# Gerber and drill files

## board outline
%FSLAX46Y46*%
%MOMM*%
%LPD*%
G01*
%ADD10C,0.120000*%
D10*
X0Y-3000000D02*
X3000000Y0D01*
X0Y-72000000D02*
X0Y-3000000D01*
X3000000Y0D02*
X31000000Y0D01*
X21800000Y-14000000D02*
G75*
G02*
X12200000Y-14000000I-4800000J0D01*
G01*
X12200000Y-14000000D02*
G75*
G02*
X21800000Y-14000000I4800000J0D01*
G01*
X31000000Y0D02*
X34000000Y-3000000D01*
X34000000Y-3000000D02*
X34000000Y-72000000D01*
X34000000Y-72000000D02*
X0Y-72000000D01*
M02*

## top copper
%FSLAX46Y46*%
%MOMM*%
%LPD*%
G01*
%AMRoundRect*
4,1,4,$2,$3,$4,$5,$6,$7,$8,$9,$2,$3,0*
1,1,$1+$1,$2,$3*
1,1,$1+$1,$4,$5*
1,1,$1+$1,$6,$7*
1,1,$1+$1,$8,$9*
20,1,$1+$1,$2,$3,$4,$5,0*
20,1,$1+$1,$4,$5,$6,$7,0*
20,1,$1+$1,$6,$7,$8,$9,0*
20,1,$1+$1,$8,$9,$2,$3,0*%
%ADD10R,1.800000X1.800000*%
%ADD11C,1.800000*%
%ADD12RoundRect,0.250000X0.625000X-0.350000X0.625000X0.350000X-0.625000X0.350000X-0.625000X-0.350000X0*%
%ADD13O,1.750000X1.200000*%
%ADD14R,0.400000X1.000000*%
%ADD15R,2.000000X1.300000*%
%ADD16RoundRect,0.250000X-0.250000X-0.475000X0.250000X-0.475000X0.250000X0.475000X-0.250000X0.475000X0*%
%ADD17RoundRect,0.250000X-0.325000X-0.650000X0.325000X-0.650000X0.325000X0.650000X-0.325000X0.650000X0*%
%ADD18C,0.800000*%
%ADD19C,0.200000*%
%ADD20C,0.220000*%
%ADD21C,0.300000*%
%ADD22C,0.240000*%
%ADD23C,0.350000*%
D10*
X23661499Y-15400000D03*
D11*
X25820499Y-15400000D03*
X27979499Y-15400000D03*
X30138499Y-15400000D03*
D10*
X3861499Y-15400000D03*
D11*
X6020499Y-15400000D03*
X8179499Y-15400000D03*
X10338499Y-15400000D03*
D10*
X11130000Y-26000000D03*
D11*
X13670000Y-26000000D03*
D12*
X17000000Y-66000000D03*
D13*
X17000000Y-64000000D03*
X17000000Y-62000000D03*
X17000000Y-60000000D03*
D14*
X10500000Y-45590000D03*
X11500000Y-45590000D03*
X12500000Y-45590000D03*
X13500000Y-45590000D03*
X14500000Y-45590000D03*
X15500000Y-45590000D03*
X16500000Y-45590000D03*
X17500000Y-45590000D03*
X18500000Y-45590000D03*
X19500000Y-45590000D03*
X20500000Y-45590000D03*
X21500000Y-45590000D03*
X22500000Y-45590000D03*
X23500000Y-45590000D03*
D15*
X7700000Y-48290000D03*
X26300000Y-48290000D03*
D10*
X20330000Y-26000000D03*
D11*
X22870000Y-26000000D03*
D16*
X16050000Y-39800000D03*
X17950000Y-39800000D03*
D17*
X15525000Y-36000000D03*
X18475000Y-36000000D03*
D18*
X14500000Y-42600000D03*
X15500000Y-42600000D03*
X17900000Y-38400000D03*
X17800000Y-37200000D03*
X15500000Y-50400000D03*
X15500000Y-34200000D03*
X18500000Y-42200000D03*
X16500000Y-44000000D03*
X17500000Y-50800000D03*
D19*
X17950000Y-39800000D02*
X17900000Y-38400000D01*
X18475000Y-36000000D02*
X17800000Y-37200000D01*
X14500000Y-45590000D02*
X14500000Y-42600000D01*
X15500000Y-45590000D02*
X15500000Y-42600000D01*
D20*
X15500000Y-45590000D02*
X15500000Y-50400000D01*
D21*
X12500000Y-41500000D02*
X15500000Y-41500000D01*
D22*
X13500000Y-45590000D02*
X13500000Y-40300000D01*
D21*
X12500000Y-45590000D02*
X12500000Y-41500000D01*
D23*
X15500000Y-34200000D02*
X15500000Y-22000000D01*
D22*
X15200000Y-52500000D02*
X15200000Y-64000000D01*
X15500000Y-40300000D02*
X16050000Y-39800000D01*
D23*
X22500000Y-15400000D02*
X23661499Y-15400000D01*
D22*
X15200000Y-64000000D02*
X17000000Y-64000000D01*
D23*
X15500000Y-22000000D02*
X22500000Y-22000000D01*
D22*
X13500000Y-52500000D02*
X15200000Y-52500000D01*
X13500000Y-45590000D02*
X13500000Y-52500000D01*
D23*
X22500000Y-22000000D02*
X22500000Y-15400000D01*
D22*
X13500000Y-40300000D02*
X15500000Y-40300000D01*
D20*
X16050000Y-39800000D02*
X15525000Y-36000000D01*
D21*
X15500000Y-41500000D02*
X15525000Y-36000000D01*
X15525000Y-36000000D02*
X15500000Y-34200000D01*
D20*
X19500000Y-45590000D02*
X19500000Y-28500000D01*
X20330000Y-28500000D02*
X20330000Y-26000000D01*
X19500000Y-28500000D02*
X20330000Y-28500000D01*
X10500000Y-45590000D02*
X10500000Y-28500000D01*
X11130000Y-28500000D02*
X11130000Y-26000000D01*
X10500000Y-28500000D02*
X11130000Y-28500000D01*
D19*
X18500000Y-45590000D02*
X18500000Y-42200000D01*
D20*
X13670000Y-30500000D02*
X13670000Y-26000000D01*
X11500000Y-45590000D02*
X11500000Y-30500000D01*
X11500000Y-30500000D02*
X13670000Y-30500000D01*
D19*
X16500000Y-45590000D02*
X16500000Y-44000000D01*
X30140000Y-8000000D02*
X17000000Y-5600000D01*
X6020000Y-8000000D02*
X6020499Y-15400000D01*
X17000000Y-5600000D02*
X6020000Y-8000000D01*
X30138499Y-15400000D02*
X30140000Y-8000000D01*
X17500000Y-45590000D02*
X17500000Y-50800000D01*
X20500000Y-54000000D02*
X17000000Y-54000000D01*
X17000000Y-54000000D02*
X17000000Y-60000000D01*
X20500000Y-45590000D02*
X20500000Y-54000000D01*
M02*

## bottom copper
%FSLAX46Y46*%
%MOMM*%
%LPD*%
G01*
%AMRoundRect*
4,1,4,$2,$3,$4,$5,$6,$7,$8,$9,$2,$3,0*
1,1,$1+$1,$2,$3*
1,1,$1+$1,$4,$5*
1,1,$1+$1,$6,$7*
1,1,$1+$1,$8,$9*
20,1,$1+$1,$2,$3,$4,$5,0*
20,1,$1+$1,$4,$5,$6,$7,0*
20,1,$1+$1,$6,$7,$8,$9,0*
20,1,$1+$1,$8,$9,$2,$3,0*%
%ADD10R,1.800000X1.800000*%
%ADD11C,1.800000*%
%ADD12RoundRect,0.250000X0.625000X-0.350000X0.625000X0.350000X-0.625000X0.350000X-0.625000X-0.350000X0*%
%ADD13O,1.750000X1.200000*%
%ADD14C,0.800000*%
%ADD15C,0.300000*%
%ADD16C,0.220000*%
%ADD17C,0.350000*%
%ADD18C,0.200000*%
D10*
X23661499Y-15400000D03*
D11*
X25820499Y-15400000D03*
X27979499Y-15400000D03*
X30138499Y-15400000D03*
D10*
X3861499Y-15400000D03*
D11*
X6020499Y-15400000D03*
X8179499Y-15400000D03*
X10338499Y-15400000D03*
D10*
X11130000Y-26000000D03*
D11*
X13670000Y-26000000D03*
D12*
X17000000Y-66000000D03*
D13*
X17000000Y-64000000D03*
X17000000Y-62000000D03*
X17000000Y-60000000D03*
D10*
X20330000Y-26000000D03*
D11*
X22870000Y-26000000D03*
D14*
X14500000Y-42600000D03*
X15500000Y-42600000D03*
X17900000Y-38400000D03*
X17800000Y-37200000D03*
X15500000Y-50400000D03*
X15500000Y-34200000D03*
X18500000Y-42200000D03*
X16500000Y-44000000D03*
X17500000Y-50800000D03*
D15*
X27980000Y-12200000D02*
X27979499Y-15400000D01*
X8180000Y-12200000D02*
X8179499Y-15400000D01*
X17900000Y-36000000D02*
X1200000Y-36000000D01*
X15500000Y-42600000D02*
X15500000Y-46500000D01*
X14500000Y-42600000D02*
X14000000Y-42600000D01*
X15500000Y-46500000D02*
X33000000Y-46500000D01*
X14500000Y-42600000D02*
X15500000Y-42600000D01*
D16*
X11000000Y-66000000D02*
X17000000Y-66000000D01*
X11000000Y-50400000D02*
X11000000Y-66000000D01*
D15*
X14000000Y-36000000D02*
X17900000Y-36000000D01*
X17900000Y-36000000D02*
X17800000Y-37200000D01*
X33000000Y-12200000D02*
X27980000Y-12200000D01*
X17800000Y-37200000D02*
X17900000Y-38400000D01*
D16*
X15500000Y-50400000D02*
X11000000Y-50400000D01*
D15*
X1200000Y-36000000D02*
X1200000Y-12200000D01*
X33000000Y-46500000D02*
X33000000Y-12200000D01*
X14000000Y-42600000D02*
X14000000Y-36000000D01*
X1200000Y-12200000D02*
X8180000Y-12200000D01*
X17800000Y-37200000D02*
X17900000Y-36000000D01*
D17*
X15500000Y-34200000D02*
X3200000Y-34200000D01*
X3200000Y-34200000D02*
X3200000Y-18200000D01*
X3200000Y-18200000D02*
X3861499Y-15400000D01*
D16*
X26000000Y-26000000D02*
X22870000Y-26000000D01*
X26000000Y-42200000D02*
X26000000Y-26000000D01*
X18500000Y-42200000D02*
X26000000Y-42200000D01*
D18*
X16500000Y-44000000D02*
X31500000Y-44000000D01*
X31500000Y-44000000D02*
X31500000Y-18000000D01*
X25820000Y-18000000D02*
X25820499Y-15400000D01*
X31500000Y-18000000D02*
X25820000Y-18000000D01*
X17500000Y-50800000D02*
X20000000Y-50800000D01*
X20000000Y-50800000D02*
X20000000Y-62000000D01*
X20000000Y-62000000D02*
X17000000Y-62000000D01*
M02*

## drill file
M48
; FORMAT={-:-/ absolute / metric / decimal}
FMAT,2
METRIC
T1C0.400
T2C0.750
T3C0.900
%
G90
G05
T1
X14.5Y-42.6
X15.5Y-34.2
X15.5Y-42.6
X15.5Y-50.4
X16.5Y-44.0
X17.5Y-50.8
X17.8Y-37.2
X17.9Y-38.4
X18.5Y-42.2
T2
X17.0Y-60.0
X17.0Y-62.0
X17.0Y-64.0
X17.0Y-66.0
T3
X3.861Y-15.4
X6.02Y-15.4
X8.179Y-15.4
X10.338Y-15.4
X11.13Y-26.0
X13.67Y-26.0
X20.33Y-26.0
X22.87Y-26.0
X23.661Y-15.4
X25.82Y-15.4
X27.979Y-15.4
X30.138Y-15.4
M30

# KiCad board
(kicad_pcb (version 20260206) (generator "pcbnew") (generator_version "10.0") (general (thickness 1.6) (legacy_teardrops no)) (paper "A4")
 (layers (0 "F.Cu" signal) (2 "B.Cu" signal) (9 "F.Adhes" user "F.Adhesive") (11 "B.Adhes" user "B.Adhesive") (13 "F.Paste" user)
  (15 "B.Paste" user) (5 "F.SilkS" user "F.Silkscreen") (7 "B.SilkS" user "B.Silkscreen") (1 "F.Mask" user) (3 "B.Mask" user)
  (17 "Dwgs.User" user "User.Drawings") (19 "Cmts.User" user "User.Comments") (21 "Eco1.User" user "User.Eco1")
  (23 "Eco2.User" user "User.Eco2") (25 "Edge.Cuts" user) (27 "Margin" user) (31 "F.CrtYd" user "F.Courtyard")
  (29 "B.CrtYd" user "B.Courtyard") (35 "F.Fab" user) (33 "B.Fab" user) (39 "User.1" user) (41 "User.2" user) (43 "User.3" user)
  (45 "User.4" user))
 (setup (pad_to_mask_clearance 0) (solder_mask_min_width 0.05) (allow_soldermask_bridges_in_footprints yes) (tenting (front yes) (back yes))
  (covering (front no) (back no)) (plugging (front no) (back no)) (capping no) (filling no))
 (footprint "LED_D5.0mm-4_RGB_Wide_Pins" (layer "F.Cu") (at 23.661499 15.4)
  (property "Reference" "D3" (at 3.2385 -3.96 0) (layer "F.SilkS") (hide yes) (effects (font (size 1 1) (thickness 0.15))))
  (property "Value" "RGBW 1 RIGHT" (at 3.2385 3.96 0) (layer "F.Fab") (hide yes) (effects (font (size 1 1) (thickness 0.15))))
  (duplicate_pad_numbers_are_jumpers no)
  (pad "1" thru_hole rect (at 0 0) (size 1.8 1.8) (drill 0.9) (layers "*.Cu" "*.Mask") (remove_unused_layers no) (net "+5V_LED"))
  (pad "2" thru_hole circle (at 2.159 0) (size 1.8 1.8) (drill 0.9) (layers "*.Cu" "*.Mask") (remove_unused_layers no) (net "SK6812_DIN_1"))
  (pad "3" thru_hole circle (at 4.318 0) (size 1.8 1.8) (drill 0.9) (layers "*.Cu" "*.Mask") (remove_unused_layers no) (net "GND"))
  (pad "4" thru_hole circle (at 6.477 0) (size 1.8 1.8) (drill 0.9) (layers "*.Cu" "*.Mask") (remove_unused_layers no) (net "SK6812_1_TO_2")))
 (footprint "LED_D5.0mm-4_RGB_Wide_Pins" (layer "F.Cu") (at 3.861499 15.4)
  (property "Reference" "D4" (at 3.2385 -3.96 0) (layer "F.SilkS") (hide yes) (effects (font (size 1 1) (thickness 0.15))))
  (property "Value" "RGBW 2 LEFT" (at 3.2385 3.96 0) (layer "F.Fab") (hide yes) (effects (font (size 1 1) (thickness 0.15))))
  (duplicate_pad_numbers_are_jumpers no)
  (pad "1" thru_hole rect (at 0 0) (size 1.8 1.8) (drill 0.9) (layers "*.Cu" "*.Mask") (remove_unused_layers no) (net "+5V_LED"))
  (pad "2" thru_hole circle (at 2.159 0) (size 1.8 1.8) (drill 0.9) (layers "*.Cu" "*.Mask") (remove_unused_layers no) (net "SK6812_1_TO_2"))
  (pad "3" thru_hole circle (at 4.318 0) (size 1.8 1.8) (drill 0.9) (layers "*.Cu" "*.Mask") (remove_unused_layers no) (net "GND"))
  (pad "4" thru_hole circle (at 6.477 0) (size 1.8 1.8) (drill 0.9) (layers "*.Cu" "*.Mask") (remove_unused_layers no)))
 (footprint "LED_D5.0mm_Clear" (layer "F.Cu") (at 11.13 26)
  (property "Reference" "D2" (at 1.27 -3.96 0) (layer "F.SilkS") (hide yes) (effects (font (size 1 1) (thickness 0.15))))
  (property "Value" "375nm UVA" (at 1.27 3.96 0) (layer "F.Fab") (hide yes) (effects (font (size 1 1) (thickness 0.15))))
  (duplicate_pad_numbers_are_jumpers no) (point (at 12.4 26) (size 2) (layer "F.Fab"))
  (pad "1" thru_hole rect (at 0 0) (size 1.8 1.8) (drill 0.9) (layers "*.Cu" "*.Mask") (remove_unused_layers no) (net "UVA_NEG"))
  (pad "2" thru_hole circle (at 2.54 0) (size 1.8 1.8) (drill 0.9) (layers "*.Cu" "*.Mask") (remove_unused_layers no) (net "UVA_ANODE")))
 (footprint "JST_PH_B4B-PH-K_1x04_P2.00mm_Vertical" (layer "F.Cu") (at 17 66 90)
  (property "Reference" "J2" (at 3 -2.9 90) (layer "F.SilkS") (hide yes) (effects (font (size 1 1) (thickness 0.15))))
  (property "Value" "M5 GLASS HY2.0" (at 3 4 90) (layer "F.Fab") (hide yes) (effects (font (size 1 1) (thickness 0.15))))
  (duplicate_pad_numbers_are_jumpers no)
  (pad "1" thru_hole roundrect (at 0 0 90) (size 1.2 1.75) (drill 0.75) (layers "*.Cu" "*.Mask") (remove_unused_layers no)
   (roundrect_rratio 0.208333) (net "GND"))
  (pad "2" thru_hole oval (at 2 0 90) (size 1.2 1.75) (drill 0.75) (layers "*.Cu" "*.Mask") (remove_unused_layers no) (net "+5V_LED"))
  (pad "3" thru_hole oval (at 4 0 90) (size 1.2 1.75) (drill 0.75) (layers "*.Cu" "*.Mask") (remove_unused_layers no) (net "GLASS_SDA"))
  (pad "4" thru_hole oval (at 6 0 90) (size 1.2 1.75) (drill 0.75) (layers "*.Cu" "*.Mask") (remove_unused_layers no) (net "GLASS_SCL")))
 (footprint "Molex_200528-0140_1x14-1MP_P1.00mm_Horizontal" (layer "F.Cu") (at 17 46.5)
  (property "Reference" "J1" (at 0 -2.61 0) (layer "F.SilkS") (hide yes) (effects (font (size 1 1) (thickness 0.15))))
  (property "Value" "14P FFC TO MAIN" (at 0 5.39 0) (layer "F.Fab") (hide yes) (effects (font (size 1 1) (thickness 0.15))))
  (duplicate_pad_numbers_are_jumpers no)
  (pad "1" smd rect (at -6.5 -0.91) (size 0.4 1) (layers "F.Cu" "F.Mask" "F.Paste") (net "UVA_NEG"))
  (pad "2" smd rect (at -5.5 -0.91) (size 0.4 1) (layers "F.Cu" "F.Mask" "F.Paste") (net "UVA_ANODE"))
  (pad "3" smd rect (at -4.5 -0.91) (size 0.4 1) (layers "F.Cu" "F.Mask" "F.Paste") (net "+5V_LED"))
  (pad "4" smd rect (at -3.5 -0.91) (size 0.4 1) (layers "F.Cu" "F.Mask" "F.Paste") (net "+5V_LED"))
  (pad "5" smd rect (at -2.5 -0.91) (size 0.4 1) (layers "F.Cu" "F.Mask" "F.Paste") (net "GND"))
  (pad "6" smd rect (at -1.5 -0.91) (size 0.4 1) (layers "F.Cu" "F.Mask" "F.Paste") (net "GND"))
  (pad "7" smd rect (at -0.5 -0.91) (size 0.4 1) (layers "F.Cu" "F.Mask" "F.Paste") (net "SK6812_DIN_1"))
  (pad "8" smd rect (at 0.5 -0.91) (size 0.4 1) (layers "F.Cu" "F.Mask" "F.Paste") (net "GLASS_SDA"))
  (pad "9" smd rect (at 1.5 -0.91) (size 0.4 1) (layers "F.Cu" "F.Mask" "F.Paste") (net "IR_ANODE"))
  (pad "10" smd rect (at 2.5 -0.91) (size 0.4 1) (layers "F.Cu" "F.Mask" "F.Paste") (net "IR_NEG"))
  (pad "11" smd rect (at 3.5 -0.91) (size 0.4 1) (layers "F.Cu" "F.Mask" "F.Paste") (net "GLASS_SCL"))
  (pad "12" smd rect (at 4.5 -0.91) (size 0.4 1) (layers "F.Cu" "F.Mask" "F.Paste"))
  (pad "13" smd rect (at 5.5 -0.91) (size 0.4 1) (layers "F.Cu" "F.Mask" "F.Paste"))
  (pad "14" smd rect (at 6.5 -0.91) (size 0.4 1) (layers "F.Cu" "F.Mask" "F.Paste"))
  (pad "MP" smd rect (at -9.3 1.79) (size 2 1.3) (layers "F.Cu" "F.Mask" "F.Paste"))
  (pad "MP" smd rect (at 9.3 1.79) (size 2 1.3) (layers "F.Cu" "F.Mask" "F.Paste")))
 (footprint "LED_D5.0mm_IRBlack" (layer "F.Cu") (at 20.33 26)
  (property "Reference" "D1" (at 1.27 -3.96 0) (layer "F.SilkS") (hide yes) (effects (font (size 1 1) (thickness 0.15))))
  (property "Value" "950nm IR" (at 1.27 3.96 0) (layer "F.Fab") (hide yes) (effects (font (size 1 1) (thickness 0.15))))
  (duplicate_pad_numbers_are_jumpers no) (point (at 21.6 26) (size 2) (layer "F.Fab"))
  (pad "1" thru_hole rect (at 0 0) (size 1.8 1.8) (drill 0.9) (layers "*.Cu" "*.Mask") (remove_unused_layers no) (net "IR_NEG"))
  (pad "2" thru_hole circle (at 2.54 0) (size 1.8 1.8) (drill 0.9) (layers "*.Cu" "*.Mask") (remove_unused_layers no) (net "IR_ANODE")))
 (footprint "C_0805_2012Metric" (layer "F.Cu") (at 17 39.8)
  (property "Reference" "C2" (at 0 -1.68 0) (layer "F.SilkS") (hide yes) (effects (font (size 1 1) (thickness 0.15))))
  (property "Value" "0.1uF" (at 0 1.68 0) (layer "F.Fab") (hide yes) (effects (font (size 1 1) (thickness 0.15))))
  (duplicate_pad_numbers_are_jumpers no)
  (pad "1" smd roundrect (at -0.95 0) (size 1 1.45) (layers "F.Cu" "F.Mask" "F.Paste") (roundrect_rratio 0.25) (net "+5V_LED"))
  (pad "2" smd roundrect (at 0.95 0) (size 1 1.45) (layers "F.Cu" "F.Mask" "F.Paste") (roundrect_rratio 0.25) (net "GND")))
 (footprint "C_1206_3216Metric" (layer "F.Cu") (at 17 36)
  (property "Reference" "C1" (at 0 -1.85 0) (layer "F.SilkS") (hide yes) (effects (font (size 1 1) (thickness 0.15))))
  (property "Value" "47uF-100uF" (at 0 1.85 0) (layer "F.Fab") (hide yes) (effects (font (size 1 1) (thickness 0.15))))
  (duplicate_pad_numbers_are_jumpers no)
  (pad "1" smd roundrect (at -1.475 0) (size 1.15 1.8) (layers "F.Cu" "F.Mask" "F.Paste") (roundrect_rratio 0.217391) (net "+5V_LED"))
  (pad "2" smd roundrect (at 1.475 0) (size 1.15 1.8) (layers "F.Cu" "F.Mask" "F.Paste") (roundrect_rratio 0.217391) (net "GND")))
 (gr_line (start 0 3) (end 3 0) (stroke (width 0.12) (type default)) (layer "Edge.Cuts"))
 (gr_line (start 0 72) (end 0 3) (stroke (width 0.12) (type default)) (layer "Edge.Cuts"))
 (gr_line (start 3 0) (end 31 0) (stroke (width 0.12) (type default)) (layer "Edge.Cuts"))
 (gr_circle (center 17 14) (end 21.8 14) (stroke (width 0.12) (type default)) (fill no) (layer "Edge.Cuts"))
 (gr_line (start 31 0) (end 34 3) (stroke (width 0.12) (type default)) (layer "Edge.Cuts"))
 (gr_line (start 34 3) (end 34 72) (stroke (width 0.12) (type default)) (layer "Edge.Cuts"))
 (gr_line (start 34 72) (end 0 72) (stroke (width 0.12) (type default)) (layer "Edge.Cuts"))
 (segment (start 17.95 39.8) (end 17.9 38.4) (width 0.2) (layer "F.Cu") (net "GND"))
 (segment (start 18.475 36) (end 17.8 37.2) (width 0.2) (layer "F.Cu") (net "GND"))
 (segment (start 14.5 45.59) (end 14.5 42.6) (width 0.2) (layer "F.Cu") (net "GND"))
 (segment (start 15.5 45.59) (end 15.5 42.6) (width 0.2) (layer "F.Cu") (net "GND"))
 (segment (start 15.5 45.59) (end 15.5 50.4) (width 0.22) (layer "F.Cu") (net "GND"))
 (via (at 14.5 42.6) (size 0.8) (drill 0.4) (layers "F.Cu" "B.Cu") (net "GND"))
 (via (at 15.5 42.6) (size 0.8) (drill 0.4) (layers "F.Cu" "B.Cu") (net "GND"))
 (via (at 17.9 38.4) (size 0.8) (drill 0.4) (layers "F.Cu" "B.Cu") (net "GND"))
 (via (at 17.8 37.2) (size 0.8) (drill 0.4) (layers "F.Cu" "B.Cu") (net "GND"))
 (via (at 15.5 50.4) (size 0.8) (drill 0.4) (layers "F.Cu" "B.Cu") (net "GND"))
 (segment (start 27.98 12.2) (end 27.979499 15.4) (width 0.3) (layer "B.Cu") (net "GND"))
 (segment (start 8.18 12.2) (end 8.179499 15.4) (width 0.3) (layer "B.Cu") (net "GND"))
 (segment (start 17.9 36) (end 1.2 36) (width 0.3) (layer "B.Cu") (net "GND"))
 (segment (start 15.5 42.6) (end 15.5 46.5) (width 0.3) (layer "B.Cu") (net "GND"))
 (segment (start 14.5 42.6) (end 14 42.6) (width 0.3) (layer "B.Cu") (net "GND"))
 (segment (start 15.5 46.5) (end 33 46.5) (width 0.3) (layer "B.Cu") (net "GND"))
 (segment (start 14.5 42.6) (end 15.5 42.6) (width 0.3) (layer "B.Cu") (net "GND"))
 (segment (start 11 66) (end 17 66) (width 0.22) (layer "B.Cu") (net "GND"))
 (segment (start 11 50.4) (end 11 66) (width 0.22) (layer "B.Cu") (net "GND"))
 (segment (start 14 36) (end 17.9 36) (width 0.3) (layer "B.Cu") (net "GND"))
 (segment (start 17.9 36) (end 17.8 37.2) (width 0.3) (layer "B.Cu") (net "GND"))
 (segment (start 33 12.2) (end 27.98 12.2) (width 0.3) (layer "B.Cu") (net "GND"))
 (segment (start 17.8 37.2) (end 17.9 38.4) (width 0.3) (layer "B.Cu") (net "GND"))
 (segment (start 15.5 50.4) (end 11 50.4) (width 0.22) (layer "B.Cu") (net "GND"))
 (segment (start 1.2 36) (end 1.2 12.2) (width 0.3) (layer "B.Cu") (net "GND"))
 (segment (start 33 46.5) (end 33 12.2) (width 0.3) (layer "B.Cu") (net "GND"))
 (segment (start 14 42.6) (end 14 36) (width 0.3) (layer "B.Cu") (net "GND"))
 (segment (start 1.2 12.2) (end 8.18 12.2) (width 0.3) (layer "B.Cu") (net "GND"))
 (segment (start 17.8 37.2) (end 17.9 36) (width 0.3) (layer "B.Cu") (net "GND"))
 (segment (start 12.5 41.5) (end 15.5 41.5) (width 0.3) (layer "F.Cu") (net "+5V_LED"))
 (segment (start 13.5 45.59) (end 13.5 40.3) (width 0.24) (layer "F.Cu") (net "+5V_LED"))
 (segment (start 12.5 45.59) (end 12.5 41.5) (width 0.3) (layer "F.Cu") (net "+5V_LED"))
 (segment (start 15.5 34.2) (end 15.5 22) (width 0.35) (layer "F.Cu") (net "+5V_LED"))
 (segment (start 15.2 52.5) (end 15.2 64) (width 0.24) (layer "F.Cu") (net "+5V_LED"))
 (segment (start 15.5 40.3) (end 16.05 39.8) (width 0.24) (layer "F.Cu") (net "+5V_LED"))
 (segment (start 22.5 15.4) (end 23.661499 15.4) (width 0.35) (layer "F.Cu") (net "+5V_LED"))
 (segment (start 15.2 64) (end 17 64) (width 0.24) (layer "F.Cu") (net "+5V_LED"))
 (segment (start 15.5 22) (end 22.5 22) (width 0.35) (layer "F.Cu") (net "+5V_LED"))
 (segment (start 13.5 52.5) (end 15.2 52.5) (width 0.24) (layer "F.Cu") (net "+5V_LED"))
 (segment (start 13.5 45.59) (end 13.5 52.5) (width 0.24) (layer "F.Cu") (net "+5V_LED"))
 (segment (start 22.5 22) (end 22.5 15.4) (width 0.35) (layer "F.Cu") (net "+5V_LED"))
 (segment (start 13.5 40.3) (end 15.5 40.3) (width 0.24) (layer "F.Cu") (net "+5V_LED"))
 (segment (start 16.05 39.8) (end 15.525 36) (width 0.22) (layer "F.Cu") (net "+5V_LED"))
 (segment (start 15.5 41.5) (end 15.525 36) (width 0.3) (layer "F.Cu") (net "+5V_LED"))
 (segment (start 15.525 36) (end 15.5 34.2) (width 0.3) (layer "F.Cu") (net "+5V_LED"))
 (via (at 15.5 34.2) (size 0.8) (drill 0.4) (layers "F.Cu" "B.Cu") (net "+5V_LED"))
 (segment (start 15.5 34.2) (end 3.2 34.2) (width 0.35) (layer "B.Cu") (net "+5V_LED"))
 (segment (start 3.2 34.2) (end 3.2 18.2) (width 0.35) (layer "B.Cu") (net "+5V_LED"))
 (segment (start 3.2 18.2) (end 3.861499 15.4) (width 0.35) (layer "B.Cu") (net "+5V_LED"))
 (segment (start 19.5 45.59) (end 19.5 28.5) (width 0.22) (layer "F.Cu") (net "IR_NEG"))
 (segment (start 20.33 28.5) (end 20.33 26) (width 0.22) (layer "F.Cu") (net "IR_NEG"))
 (segment (start 19.5 28.5) (end 20.33 28.5) (width 0.22) (layer "F.Cu") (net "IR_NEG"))
 (segment (start 10.5 45.59) (end 10.5 28.5) (width 0.22) (layer "F.Cu") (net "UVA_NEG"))
 (segment (start 11.13 28.5) (end 11.13 26) (width 0.22) (layer "F.Cu") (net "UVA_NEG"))
 (segment (start 10.5 28.5) (end 11.13 28.5) (width 0.22) (layer "F.Cu") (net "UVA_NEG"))
 (segment (start 18.5 45.59) (end 18.5 42.2) (width 0.2) (layer "F.Cu") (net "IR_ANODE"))
 (via (at 18.5 42.2) (size 0.8) (drill 0.4) (layers "F.Cu" "B.Cu") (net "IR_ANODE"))
 (segment (start 26 26) (end 22.87 26) (width 0.22) (layer "B.Cu") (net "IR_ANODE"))
 (segment (start 26 42.2) (end 26 26) (width 0.22) (layer "B.Cu") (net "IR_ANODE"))
 (segment (start 18.5 42.2) (end 26 42.2) (width 0.22) (layer "B.Cu") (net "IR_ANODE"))
 (segment (start 13.67 30.5) (end 13.67 26) (width 0.22) (layer "F.Cu") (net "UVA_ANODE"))
 (segment (start 11.5 45.59) (end 11.5 30.5) (width 0.22) (layer "F.Cu") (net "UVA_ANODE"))
 (segment (start 11.5 30.5) (end 13.67 30.5) (width 0.22) (layer "F.Cu") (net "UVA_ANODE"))
 (segment (start 16.5 45.59) (end 16.5 44) (width 0.2) (layer "F.Cu") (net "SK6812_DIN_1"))
 (via (at 16.5 44) (size 0.8) (drill 0.4) (layers "F.Cu" "B.Cu") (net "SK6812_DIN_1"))
 (segment (start 16.5 44) (end 31.5 44) (width 0.2) (layer "B.Cu") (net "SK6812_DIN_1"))
 (segment (start 31.5 44) (end 31.5 18) (width 0.2) (layer "B.Cu") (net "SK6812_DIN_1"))
 (segment (start 25.82 18) (end 25.820499 15.4) (width 0.2) (layer "B.Cu") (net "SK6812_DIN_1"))
 (segment (start 31.5 18) (end 25.82 18) (width 0.2) (layer "B.Cu") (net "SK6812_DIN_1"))
 (segment (start 30.14 8) (end 17 5.6) (width 0.2) (layer "F.Cu") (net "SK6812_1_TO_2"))
 (segment (start 6.02 8) (end 6.020499 15.4) (width 0.2) (layer "F.Cu") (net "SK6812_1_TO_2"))
 (segment (start 17 5.6) (end 6.02 8) (width 0.2) (layer "F.Cu") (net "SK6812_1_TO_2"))
 (segment (start 30.138499 15.4) (end 30.14 8) (width 0.2) (layer "F.Cu") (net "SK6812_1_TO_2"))
 (segment (start 17.5 45.59) (end 17.5 50.8) (width 0.2) (layer "F.Cu") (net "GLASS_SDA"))
 (via (at 17.5 50.8) (size 0.8) (drill 0.4) (layers "F.Cu" "B.Cu") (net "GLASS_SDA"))
 (segment (start 17.5 50.8) (end 20 50.8) (width 0.2) (layer "B.Cu") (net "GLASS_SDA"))
 (segment (start 20 50.8) (end 20 62) (width 0.2) (layer "B.Cu") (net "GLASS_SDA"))
 (segment (start 20 62) (end 17 62) (width 0.2) (layer "B.Cu") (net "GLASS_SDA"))
 (segment (start 20.5 54) (end 17 54) (width 0.2) (layer "F.Cu") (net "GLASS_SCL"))
 (segment (start 17 54) (end 17 60) (width 0.2) (layer "F.Cu") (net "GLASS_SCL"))
 (segment (start 20.5 45.59) (end 20.5 54) (width 0.2) (layer "F.Cu") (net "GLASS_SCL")))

